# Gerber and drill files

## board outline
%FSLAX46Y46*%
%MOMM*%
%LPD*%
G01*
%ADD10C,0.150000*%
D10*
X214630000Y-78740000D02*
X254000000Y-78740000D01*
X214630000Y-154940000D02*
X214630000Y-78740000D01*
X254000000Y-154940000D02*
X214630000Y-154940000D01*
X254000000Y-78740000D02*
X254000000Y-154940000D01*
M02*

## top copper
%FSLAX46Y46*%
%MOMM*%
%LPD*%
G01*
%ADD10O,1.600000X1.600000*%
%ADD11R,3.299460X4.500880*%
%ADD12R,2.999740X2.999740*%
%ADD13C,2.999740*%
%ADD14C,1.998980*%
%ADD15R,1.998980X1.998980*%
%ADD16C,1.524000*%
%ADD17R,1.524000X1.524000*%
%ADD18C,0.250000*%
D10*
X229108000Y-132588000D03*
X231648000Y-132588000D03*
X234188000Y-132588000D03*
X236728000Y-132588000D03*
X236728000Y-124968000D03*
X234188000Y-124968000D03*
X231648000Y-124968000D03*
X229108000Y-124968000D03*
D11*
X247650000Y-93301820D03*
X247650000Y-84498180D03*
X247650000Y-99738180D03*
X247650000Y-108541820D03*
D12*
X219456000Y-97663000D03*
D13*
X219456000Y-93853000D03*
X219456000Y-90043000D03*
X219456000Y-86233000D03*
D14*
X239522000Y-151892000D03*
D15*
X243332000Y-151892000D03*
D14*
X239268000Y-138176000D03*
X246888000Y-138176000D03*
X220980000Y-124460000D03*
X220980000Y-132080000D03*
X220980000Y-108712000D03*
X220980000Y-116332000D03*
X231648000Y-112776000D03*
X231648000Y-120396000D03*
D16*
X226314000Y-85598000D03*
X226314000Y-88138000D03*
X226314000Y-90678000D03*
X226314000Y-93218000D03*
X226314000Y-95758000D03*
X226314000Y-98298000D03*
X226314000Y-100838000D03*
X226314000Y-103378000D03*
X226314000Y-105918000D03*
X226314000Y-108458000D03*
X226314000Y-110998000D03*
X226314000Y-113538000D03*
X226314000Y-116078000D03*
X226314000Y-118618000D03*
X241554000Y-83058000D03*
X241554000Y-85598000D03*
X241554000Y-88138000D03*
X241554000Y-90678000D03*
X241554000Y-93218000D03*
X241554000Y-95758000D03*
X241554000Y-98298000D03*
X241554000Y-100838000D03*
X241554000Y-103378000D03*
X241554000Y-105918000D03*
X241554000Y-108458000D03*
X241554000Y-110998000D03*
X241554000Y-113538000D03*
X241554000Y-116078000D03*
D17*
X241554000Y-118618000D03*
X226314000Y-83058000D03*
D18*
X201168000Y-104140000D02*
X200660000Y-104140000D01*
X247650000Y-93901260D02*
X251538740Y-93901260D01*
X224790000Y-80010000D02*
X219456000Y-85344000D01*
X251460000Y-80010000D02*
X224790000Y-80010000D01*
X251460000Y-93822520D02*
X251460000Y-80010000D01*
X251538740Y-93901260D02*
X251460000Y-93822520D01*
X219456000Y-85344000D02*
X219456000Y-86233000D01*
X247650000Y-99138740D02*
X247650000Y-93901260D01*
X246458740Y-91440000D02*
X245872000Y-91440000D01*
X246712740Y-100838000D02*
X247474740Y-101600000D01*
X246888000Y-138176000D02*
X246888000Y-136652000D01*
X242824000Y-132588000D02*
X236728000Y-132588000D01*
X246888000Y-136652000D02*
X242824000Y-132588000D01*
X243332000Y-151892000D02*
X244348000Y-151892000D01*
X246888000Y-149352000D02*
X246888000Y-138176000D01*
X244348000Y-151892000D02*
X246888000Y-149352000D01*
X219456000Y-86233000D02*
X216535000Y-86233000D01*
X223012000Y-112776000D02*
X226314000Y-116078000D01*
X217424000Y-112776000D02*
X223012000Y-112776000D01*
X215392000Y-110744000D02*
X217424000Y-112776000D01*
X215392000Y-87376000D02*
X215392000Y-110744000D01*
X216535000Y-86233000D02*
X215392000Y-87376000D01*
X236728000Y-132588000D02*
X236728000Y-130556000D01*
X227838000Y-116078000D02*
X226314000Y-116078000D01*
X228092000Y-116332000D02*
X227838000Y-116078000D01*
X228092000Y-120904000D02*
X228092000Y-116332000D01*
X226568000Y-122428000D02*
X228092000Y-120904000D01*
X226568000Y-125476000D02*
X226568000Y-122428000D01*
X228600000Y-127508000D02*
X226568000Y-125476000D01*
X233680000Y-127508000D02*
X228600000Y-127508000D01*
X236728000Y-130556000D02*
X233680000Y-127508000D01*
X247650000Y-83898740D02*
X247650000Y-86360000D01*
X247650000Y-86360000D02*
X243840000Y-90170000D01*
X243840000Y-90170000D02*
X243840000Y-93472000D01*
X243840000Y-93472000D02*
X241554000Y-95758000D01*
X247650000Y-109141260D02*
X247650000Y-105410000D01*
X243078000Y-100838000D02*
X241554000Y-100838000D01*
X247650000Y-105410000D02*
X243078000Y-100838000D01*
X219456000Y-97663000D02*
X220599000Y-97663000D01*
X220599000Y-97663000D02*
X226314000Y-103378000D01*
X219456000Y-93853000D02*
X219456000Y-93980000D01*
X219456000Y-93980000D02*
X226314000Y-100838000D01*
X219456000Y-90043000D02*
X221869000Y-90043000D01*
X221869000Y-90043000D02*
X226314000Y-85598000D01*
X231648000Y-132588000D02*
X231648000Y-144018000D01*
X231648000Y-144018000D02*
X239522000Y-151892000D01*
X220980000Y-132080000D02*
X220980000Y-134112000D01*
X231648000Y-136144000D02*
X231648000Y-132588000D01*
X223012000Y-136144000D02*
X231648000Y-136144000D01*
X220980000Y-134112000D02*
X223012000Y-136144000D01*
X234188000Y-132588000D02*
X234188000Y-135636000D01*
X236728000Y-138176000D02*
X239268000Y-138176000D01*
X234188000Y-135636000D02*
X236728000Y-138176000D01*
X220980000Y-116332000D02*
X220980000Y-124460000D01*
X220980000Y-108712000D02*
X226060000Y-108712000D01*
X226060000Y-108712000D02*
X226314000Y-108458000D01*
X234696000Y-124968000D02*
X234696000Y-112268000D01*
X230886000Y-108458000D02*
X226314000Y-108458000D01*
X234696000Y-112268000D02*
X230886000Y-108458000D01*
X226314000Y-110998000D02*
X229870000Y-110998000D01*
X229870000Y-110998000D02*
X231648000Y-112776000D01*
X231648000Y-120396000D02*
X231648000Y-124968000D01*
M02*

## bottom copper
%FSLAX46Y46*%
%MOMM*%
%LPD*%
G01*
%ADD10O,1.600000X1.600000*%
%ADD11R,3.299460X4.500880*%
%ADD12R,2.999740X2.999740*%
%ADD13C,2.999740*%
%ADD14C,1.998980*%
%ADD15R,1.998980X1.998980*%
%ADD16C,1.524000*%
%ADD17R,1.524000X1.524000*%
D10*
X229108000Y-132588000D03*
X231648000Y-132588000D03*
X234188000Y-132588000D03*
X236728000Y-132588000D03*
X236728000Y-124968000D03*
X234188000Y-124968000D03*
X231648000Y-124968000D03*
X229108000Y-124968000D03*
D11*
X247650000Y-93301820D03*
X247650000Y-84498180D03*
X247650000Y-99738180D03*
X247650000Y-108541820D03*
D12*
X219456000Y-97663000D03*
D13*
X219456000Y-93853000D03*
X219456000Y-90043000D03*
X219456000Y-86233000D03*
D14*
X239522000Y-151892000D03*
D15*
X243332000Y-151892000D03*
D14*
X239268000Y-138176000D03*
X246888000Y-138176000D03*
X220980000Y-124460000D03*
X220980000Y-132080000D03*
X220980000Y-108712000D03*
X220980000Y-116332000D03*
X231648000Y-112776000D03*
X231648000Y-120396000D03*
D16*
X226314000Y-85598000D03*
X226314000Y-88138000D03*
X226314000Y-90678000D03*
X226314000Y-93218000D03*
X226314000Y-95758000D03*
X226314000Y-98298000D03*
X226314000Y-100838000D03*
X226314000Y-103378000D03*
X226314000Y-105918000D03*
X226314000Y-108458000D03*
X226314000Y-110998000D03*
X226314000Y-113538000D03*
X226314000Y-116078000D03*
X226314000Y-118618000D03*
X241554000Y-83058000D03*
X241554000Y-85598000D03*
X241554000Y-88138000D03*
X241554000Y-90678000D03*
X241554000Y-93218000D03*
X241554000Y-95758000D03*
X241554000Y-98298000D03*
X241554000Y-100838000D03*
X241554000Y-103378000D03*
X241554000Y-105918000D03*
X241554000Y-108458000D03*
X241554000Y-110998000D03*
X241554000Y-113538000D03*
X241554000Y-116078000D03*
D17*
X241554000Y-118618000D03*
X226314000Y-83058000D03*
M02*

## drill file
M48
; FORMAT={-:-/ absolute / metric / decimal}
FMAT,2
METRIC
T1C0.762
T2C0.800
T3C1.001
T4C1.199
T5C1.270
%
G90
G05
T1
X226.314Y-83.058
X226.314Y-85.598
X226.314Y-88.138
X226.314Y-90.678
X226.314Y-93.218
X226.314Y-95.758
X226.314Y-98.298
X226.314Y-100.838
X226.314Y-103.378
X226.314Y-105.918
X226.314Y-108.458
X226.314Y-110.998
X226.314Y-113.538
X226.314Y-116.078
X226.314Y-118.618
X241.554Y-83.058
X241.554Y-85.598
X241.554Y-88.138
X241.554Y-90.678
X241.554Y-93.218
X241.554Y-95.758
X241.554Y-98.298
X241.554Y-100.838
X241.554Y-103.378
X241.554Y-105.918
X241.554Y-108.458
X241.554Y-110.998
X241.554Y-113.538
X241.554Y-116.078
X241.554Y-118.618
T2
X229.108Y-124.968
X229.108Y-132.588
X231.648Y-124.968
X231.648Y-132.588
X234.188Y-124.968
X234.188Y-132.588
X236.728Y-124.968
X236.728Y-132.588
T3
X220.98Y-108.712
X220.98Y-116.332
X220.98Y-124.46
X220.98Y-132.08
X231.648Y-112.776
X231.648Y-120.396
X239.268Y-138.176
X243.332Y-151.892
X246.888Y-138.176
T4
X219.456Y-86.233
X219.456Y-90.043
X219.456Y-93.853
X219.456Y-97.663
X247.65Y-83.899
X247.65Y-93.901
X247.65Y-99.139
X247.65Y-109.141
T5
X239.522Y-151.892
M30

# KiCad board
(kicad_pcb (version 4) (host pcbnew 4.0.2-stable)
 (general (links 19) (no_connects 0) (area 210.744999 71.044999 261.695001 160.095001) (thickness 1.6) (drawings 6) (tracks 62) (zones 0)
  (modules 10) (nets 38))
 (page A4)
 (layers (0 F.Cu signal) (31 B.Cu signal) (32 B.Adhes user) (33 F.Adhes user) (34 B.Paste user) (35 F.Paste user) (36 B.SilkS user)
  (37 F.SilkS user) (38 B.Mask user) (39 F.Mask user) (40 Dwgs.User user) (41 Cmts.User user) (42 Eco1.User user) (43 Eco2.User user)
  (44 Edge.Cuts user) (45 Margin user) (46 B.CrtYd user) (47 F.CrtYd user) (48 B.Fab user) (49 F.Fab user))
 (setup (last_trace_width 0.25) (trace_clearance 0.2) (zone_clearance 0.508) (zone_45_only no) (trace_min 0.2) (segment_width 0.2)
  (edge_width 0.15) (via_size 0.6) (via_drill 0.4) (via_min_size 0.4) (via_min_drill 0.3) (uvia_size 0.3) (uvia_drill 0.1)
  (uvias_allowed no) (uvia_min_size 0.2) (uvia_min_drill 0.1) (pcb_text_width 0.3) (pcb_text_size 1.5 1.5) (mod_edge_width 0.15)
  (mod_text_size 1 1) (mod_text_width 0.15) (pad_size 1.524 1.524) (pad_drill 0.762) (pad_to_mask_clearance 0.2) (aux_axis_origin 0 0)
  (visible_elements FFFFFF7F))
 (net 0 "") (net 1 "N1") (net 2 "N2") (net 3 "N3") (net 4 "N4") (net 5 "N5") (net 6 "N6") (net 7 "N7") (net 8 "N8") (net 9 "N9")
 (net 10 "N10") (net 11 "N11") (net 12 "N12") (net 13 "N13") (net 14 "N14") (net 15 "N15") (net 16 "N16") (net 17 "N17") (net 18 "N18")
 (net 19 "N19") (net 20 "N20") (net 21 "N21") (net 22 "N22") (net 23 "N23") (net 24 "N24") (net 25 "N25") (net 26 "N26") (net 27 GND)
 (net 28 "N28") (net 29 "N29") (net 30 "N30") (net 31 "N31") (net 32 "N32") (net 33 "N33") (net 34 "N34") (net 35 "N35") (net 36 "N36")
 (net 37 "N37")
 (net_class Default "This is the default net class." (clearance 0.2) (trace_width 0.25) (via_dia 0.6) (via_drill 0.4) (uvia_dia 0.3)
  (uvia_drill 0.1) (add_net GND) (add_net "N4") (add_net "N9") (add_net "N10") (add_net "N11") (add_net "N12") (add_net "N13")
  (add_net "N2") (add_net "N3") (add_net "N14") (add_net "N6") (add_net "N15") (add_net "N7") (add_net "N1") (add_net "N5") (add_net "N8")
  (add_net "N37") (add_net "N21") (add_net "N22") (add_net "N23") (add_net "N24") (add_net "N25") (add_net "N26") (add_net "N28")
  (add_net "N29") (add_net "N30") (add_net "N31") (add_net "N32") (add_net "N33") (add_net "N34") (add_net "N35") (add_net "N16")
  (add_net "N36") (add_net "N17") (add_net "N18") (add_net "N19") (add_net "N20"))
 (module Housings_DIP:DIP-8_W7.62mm (layer F.Cu) (at 229.108 132.588 90)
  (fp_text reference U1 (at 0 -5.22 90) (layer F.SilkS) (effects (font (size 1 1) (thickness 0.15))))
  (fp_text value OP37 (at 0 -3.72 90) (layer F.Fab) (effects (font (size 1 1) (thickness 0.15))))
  (pad 1 thru_hole oval (at 0 0 90) (size 1.6 1.6) (drill 0.8) (layers *.Cu *.Mask F.SilkS) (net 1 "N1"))
  (pad 2 thru_hole oval (at 0 2.54 90) (size 1.6 1.6) (drill 0.8) (layers *.Cu *.Mask F.SilkS) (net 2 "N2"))
  (pad 3 thru_hole oval (at 0 5.08 90) (size 1.6 1.6) (drill 0.8) (layers *.Cu *.Mask F.SilkS) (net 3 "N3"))
  (pad 4 thru_hole oval (at 0 7.62 90) (size 1.6 1.6) (drill 0.8) (layers *.Cu *.Mask F.SilkS) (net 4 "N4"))
  (pad 5 thru_hole oval (at 7.62 7.62 90) (size 1.6 1.6) (drill 0.8) (layers *.Cu *.Mask F.SilkS) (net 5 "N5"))
  (pad 6 thru_hole oval (at 7.62 5.08 90) (size 1.6 1.6) (drill 0.8) (layers *.Cu *.Mask F.SilkS) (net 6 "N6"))
  (pad 7 thru_hole oval (at 7.62 2.54 90) (size 1.6 1.6) (drill 0.8) (layers *.Cu *.Mask F.SilkS) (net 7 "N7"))
  (pad 8 thru_hole oval (at 7.62 0 90) (size 1.6 1.6) (drill 0.8) (layers *.Cu *.Mask F.SilkS) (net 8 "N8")))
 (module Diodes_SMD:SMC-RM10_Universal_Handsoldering (layer F.Cu) (at 247.65 88.9 90)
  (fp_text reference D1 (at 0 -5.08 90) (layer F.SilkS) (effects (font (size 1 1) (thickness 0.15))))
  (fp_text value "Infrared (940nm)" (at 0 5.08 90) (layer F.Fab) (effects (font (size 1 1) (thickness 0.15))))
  (pad 1 thru_hole rect (at -5.00126 0 90) (size 4.50088 3.29946) (drill 1.19888 (offset 0.59944 0)) (layers *.Cu *.Mask F.SilkS)
   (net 4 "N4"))
  (pad 2 thru_hole rect (at 5.00126 0 270) (size 4.50088 3.29946) (drill 1.19888 (offset 0.59944 0)) (layers *.Cu *.Mask F.SilkS)
   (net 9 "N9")))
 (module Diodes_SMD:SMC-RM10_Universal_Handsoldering (layer F.Cu) (at 247.65 104.14 270)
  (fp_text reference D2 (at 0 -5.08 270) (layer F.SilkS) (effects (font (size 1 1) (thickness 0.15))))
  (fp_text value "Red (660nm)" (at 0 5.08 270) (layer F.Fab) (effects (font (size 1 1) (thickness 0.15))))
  (pad 1 thru_hole rect (at -5.00126 0 270) (size 4.50088 3.29946) (drill 1.19888 (offset 0.59944 0)) (layers *.Cu *.Mask F.SilkS)
   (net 4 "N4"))
  (pad 2 thru_hole rect (at 5.00126 0 90) (size 4.50088 3.29946) (drill 1.19888 (offset 0.59944 0)) (layers *.Cu *.Mask F.SilkS)
   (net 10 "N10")))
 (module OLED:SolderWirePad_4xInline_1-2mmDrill (layer F.Cu) (at 219.456 91.948 90)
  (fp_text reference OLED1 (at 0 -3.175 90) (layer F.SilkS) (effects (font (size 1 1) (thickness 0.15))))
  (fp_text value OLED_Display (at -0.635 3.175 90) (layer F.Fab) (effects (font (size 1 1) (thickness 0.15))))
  (pad 1 thru_hole rect (at -5.715 0 90) (size 2.99974 2.99974) (drill 1.19888) (layers *.Cu *.Mask F.SilkS) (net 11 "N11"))
  (pad 2 thru_hole circle (at -1.905 0 90) (size 2.99974 2.99974) (drill 1.19888) (layers *.Cu *.Mask F.SilkS) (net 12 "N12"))
  (pad 3 thru_hole circle (at 1.905 0 90) (size 2.99974 2.99974) (drill 1.19888) (layers *.Cu *.Mask F.SilkS) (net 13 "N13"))
  (pad 4 thru_hole circle (at 5.715 0 90) (size 2.99974 2.99974) (drill 1.19888) (layers *.Cu *.Mask F.SilkS) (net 4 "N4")))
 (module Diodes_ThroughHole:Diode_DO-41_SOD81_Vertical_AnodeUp (layer F.Cu) (at 243.332 151.892 180)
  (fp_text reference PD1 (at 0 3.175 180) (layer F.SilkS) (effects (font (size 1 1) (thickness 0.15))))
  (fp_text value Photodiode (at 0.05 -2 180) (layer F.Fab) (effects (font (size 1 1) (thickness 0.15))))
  (pad 2 thru_hole circle (at 3.81 0 180) (size 1.99898 1.99898) (drill 1.27) (layers *.Cu *.Mask F.SilkS) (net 2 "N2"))
  (pad 1 thru_hole rect (at 0 0 180) (size 1.99898 1.99898) (drill 1.00076) (layers *.Cu *.Mask F.SilkS) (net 4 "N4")))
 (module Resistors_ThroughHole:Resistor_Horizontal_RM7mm (layer F.Cu) (at 239.268 138.176)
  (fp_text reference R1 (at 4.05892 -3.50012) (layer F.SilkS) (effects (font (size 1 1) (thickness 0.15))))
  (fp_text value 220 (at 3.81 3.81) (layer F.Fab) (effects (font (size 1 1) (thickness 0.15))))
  (pad 1 thru_hole circle (at 0 0) (size 1.99898 1.99898) (drill 1.00076) (layers *.Cu *.SilkS *.Mask) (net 3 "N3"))
  (pad 2 thru_hole circle (at 7.62 0) (size 1.99898 1.99898) (drill 1.00076) (layers *.Cu *.SilkS *.Mask) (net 4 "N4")))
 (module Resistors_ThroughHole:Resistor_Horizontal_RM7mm (layer F.Cu) (at 220.98 124.46 270)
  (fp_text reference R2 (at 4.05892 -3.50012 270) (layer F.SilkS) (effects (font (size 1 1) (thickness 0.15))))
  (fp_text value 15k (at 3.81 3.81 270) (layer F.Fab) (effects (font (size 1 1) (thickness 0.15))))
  (pad 1 thru_hole circle (at 0 0 270) (size 1.99898 1.99898) (drill 1.00076) (layers *.Cu *.SilkS *.Mask) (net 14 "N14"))
  (pad 2 thru_hole circle (at 7.62 0 270) (size 1.99898 1.99898) (drill 1.00076) (layers *.Cu *.SilkS *.Mask) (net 2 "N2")))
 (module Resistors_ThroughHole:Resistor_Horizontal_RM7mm (layer F.Cu) (at 220.98 108.712 270)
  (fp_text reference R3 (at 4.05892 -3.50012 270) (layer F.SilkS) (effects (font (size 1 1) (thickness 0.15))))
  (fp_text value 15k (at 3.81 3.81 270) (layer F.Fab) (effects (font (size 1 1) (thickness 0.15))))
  (pad 1 thru_hole circle (at 0 0 270) (size 1.99898 1.99898) (drill 1.00076) (layers *.Cu *.SilkS *.Mask) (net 6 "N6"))
  (pad 2 thru_hole circle (at 7.62 0 270) (size 1.99898 1.99898) (drill 1.00076) (layers *.Cu *.SilkS *.Mask) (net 14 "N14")))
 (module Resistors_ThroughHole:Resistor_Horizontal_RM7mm (layer F.Cu) (at 231.648 112.776 270)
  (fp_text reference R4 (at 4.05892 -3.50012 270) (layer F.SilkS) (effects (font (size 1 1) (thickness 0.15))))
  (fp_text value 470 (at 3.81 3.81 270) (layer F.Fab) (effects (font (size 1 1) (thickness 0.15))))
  (pad 1 thru_hole circle (at 0 0 270) (size 1.99898 1.99898) (drill 1.00076) (layers *.Cu *.SilkS *.Mask) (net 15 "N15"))
  (pad 2 thru_hole circle (at 7.62 0 270) (size 1.99898 1.99898) (drill 1.00076) (layers *.Cu *.SilkS *.Mask) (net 7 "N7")))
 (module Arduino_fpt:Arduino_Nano (layer F.Cu) (at 243.332 79.248 270)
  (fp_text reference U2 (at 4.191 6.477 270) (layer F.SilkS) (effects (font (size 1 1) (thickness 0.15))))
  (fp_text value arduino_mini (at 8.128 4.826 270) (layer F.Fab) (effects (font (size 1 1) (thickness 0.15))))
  (pad 2 thru_hole circle (at 6.35 17.018 270) (size 1.524 1.524) (drill 0.762) (layers *.Cu *.Mask F.SilkS) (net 13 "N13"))
  (pad 3 thru_hole circle (at 8.89 17.018 270) (size 1.524 1.524) (drill 0.762) (layers *.Cu *.Mask F.SilkS) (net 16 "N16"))
  (pad 4 thru_hole circle (at 11.43 17.018 270) (size 1.524 1.524) (drill 0.762) (layers *.Cu *.Mask F.SilkS) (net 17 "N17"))
  (pad 5 thru_hole circle (at 13.97 17.018 270) (size 1.524 1.524) (drill 0.762) (layers *.Cu *.Mask F.SilkS) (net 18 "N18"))
  (pad 6 thru_hole circle (at 16.51 17.018 270) (size 1.524 1.524) (drill 0.762) (layers *.Cu *.Mask F.SilkS) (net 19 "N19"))
  (pad 7 thru_hole circle (at 19.05 17.018 270) (size 1.524 1.524) (drill 0.762) (layers *.Cu *.Mask F.SilkS) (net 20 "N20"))
  (pad 8 thru_hole circle (at 21.59 17.018 270) (size 1.524 1.524) (drill 0.762) (layers *.Cu *.Mask F.SilkS) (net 12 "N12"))
  (pad 9 thru_hole circle (at 24.13 17.018 270) (size 1.524 1.524) (drill 0.762) (layers *.Cu *.Mask F.SilkS) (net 11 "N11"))
  (pad 10 thru_hole circle (at 26.67 17.018 270) (size 1.524 1.524) (drill 0.762) (layers *.Cu *.Mask F.SilkS) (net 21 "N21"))
  (pad 11 thru_hole circle (at 29.21 17.018 270) (size 1.524 1.524) (drill 0.762) (layers *.Cu *.Mask F.SilkS) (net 6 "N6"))
  (pad 12 thru_hole circle (at 31.75 17.018 270) (size 1.524 1.524) (drill 0.762) (layers *.Cu *.Mask F.SilkS) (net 15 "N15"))
  (pad 13 thru_hole circle (at 34.29 17.018 270) (size 1.524 1.524) (drill 0.762) (layers *.Cu *.Mask F.SilkS) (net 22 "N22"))
  (pad 14 thru_hole circle (at 36.83 17.018 270) (size 1.524 1.524) (drill 0.762) (layers *.Cu *.Mask F.SilkS) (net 4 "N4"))
  (pad 15 thru_hole circle (at 39.37 17.018 270) (size 1.524 1.524) (drill 0.762) (layers *.Cu *.Mask F.SilkS) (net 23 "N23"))
  (pad 16 thru_hole circle (at 3.81 1.778 270) (size 1.524 1.524) (drill 0.762) (layers *.Cu *.Mask F.SilkS) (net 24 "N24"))
  (pad 17 thru_hole circle (at 6.35 1.778 270) (size 1.524 1.524) (drill 0.762) (layers *.Cu *.Mask F.SilkS) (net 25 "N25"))
  (pad 18 thru_hole circle (at 8.89 1.778 270) (size 1.524 1.524) (drill 0.762) (layers *.Cu *.Mask F.SilkS) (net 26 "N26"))
  (pad 19 thru_hole circle (at 11.43 1.778 270) (size 1.524 1.524) (drill 0.762) (layers *.Cu *.Mask F.SilkS) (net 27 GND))
  (pad 20 thru_hole circle (at 13.97 1.778 270) (size 1.524 1.524) (drill 0.762) (layers *.Cu *.Mask F.SilkS) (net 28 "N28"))
  (pad 21 thru_hole circle (at 16.51 1.778 270) (size 1.524 1.524) (drill 0.762) (layers *.Cu *.Mask F.SilkS) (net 9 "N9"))
  (pad 22 thru_hole circle (at 19.05 1.778 270) (size 1.524 1.524) (drill 0.762) (layers *.Cu *.Mask F.SilkS) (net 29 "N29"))
  (pad 23 thru_hole circle (at 21.59 1.778 270) (size 1.524 1.524) (drill 0.762) (layers *.Cu *.Mask F.SilkS) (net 10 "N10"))
  (pad 24 thru_hole circle (at 24.13 1.778 270) (size 1.524 1.524) (drill 0.762) (layers *.Cu *.Mask F.SilkS) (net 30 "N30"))
  (pad 25 thru_hole circle (at 26.67 1.778 270) (size 1.524 1.524) (drill 0.762) (layers *.Cu *.Mask F.SilkS) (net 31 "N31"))
  (pad 26 thru_hole circle (at 29.21 1.778 270) (size 1.524 1.524) (drill 0.762) (layers *.Cu *.Mask F.SilkS) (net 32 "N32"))
  (pad 27 thru_hole circle (at 31.75 1.778 270) (size 1.524 1.524) (drill 0.762) (layers *.Cu *.Mask F.SilkS) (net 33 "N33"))
  (pad 28 thru_hole circle (at 34.29 1.778 270) (size 1.524 1.524) (drill 0.762) (layers *.Cu *.Mask F.SilkS) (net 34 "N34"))
  (pad 29 thru_hole circle (at 36.83 1.778 270) (size 1.524 1.524) (drill 0.762) (layers *.Cu *.Mask F.SilkS) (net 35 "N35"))
  (pad 30 thru_hole rect (at 39.37 1.778 270) (size 1.524 1.524) (drill 0.762) (layers *.Cu *.Mask F.SilkS) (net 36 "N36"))
  (pad 1 thru_hole rect (at 3.81 17.018 270) (size 1.524 1.524) (drill 0.762) (layers *.Cu *.Mask F.SilkS) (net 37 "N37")))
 (gr_line (start 214.63 78.74) (end 254 78.74) (angle 90) (layer Edge.Cuts) (width 0.15))
 (gr_line (start 214.63 154.94) (end 214.63 78.74) (angle 90) (layer Edge.Cuts) (width 0.15))
 (gr_line (start 254 154.94) (end 214.63 154.94) (angle 90) (layer Edge.Cuts) (width 0.15))
 (gr_line (start 254 78.74) (end 254 154.94) (angle 90) (layer Edge.Cuts) (width 0.15))
 (segment (start 201.168 104.14) (end 200.66 104.14) (width 0.25) (layer F.Cu) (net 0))
 (segment (start 247.65 93.90126) (end 251.53874 93.90126) (width 0.25) (layer F.Cu) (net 4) (status 400000))
 (segment (start 224.79 80.01) (end 219.456 85.344) (width 0.25) (layer F.Cu) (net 4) (status 800000))
 (segment (start 251.46 80.01) (end 224.79 80.01) (width 0.25) (layer F.Cu) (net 4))
 (segment (start 251.46 93.82252) (end 251.46 80.01) (width 0.25) (layer F.Cu) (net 4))
 (segment (start 251.53874 93.90126) (end 251.46 93.82252) (width 0.25) (layer F.Cu) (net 4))
 (segment (start 219.456 85.344) (end 219.456 86.233) (width 0.25) (layer F.Cu) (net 4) (status C00000))
 (segment (start 247.65 99.13874) (end 247.65 93.90126) (width 0.25) (layer F.Cu) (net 4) (status C00000))
 (segment (start 246.45874 91.44) (end 245.872 91.44) (width 0.25) (layer F.Cu) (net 4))
 (segment (start 246.71274 100.838) (end 247.47474 101.6) (width 0.25) (layer F.Cu) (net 4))
 (segment (start 246.888 138.176) (end 246.888 136.652) (width 0.25) (layer F.Cu) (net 4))
 (segment (start 242.824 132.588) (end 236.728 132.588) (width 0.25) (layer F.Cu) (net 4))
 (segment (start 246.888 136.652) (end 242.824 132.588) (width 0.25) (layer F.Cu) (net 4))
 (segment (start 243.332 151.892) (end 244.348 151.892) (width 0.25) (layer F.Cu) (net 4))
 (segment (start 246.888 149.352) (end 246.888 138.176) (width 0.25) (layer F.Cu) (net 4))
 (segment (start 244.348 151.892) (end 246.888 149.352) (width 0.25) (layer F.Cu) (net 4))
 (segment (start 219.456 86.233) (end 216.535 86.233) (width 0.25) (layer F.Cu) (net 4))
 (segment (start 223.012 112.776) (end 226.314 116.078) (width 0.25) (layer F.Cu) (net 4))
 (segment (start 217.424 112.776) (end 223.012 112.776) (width 0.25) (layer F.Cu) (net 4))
 (segment (start 215.392 110.744) (end 217.424 112.776) (width 0.25) (layer F.Cu) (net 4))
 (segment (start 215.392 87.376) (end 215.392 110.744) (width 0.25) (layer F.Cu) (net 4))
 (segment (start 216.535 86.233) (end 215.392 87.376) (width 0.25) (layer F.Cu) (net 4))
 (segment (start 236.728 132.588) (end 236.728 130.556) (width 0.25) (layer F.Cu) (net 4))
 (segment (start 227.838 116.078) (end 226.314 116.078) (width 0.25) (layer F.Cu) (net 4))
 (segment (start 228.092 116.332) (end 227.838 116.078) (width 0.25) (layer F.Cu) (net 4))
 (segment (start 228.092 120.904) (end 228.092 116.332) (width 0.25) (layer F.Cu) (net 4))
 (segment (start 226.568 122.428) (end 228.092 120.904) (width 0.25) (layer F.Cu) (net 4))
 (segment (start 226.568 125.476) (end 226.568 122.428) (width 0.25) (layer F.Cu) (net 4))
 (segment (start 228.6 127.508) (end 226.568 125.476) (width 0.25) (layer F.Cu) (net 4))
 (segment (start 233.68 127.508) (end 228.6 127.508) (width 0.25) (layer F.Cu) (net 4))
 (segment (start 236.728 130.556) (end 233.68 127.508) (width 0.25) (layer F.Cu) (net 4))
 (segment (start 247.65 83.89874) (end 247.65 86.36) (width 0.25) (layer F.Cu) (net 9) (status C00000))
 (segment (start 247.65 86.36) (end 243.84 90.17) (width 0.25) (layer F.Cu) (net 9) (status 400000))
 (segment (start 243.84 90.17) (end 243.84 93.472) (width 0.25) (layer F.Cu) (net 9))
 (segment (start 243.84 93.472) (end 241.554 95.758) (width 0.25) (layer F.Cu) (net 9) (status 800000))
 (segment (start 247.65 109.14126) (end 247.65 105.41) (width 0.25) (layer F.Cu) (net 10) (status 400000))
 (segment (start 243.078 100.838) (end 241.554 100.838) (width 0.25) (layer F.Cu) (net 10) (status 800000))
 (segment (start 247.65 105.41) (end 243.078 100.838) (width 0.25) (layer F.Cu) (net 10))
 (segment (start 219.456 97.663) (end 220.599 97.663) (width 0.25) (layer F.Cu) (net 11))
 (segment (start 220.599 97.663) (end 226.314 103.378) (width 0.25) (layer F.Cu) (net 11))
 (segment (start 219.456 93.853) (end 219.456 93.98) (width 0.25) (layer F.Cu) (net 12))
 (segment (start 219.456 93.98) (end 226.314 100.838) (width 0.25) (layer F.Cu) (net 12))
 (segment (start 219.456 90.043) (end 221.869 90.043) (width 0.25) (layer F.Cu) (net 13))
 (segment (start 221.869 90.043) (end 226.314 85.598) (width 0.25) (layer F.Cu) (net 13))
 (segment (start 231.648 132.588) (end 231.648 144.018) (width 0.25) (layer F.Cu) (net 2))
 (segment (start 231.648 144.018) (end 239.522 151.892) (width 0.25) (layer F.Cu) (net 2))
 (segment (start 220.98 132.08) (end 220.98 134.112) (width 0.25) (layer F.Cu) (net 2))
 (segment (start 231.648 136.144) (end 231.648 132.588) (width 0.25) (layer F.Cu) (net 2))
 (segment (start 223.012 136.144) (end 231.648 136.144) (width 0.25) (layer F.Cu) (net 2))
 (segment (start 220.98 134.112) (end 223.012 136.144) (width 0.25) (layer F.Cu) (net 2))
 (segment (start 234.188 132.588) (end 234.188 135.636) (width 0.25) (layer F.Cu) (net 3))
 (segment (start 236.728 138.176) (end 239.268 138.176) (width 0.25) (layer F.Cu) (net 3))
 (segment (start 234.188 135.636) (end 236.728 138.176) (width 0.25) (layer F.Cu) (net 3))
 (segment (start 220.98 116.332) (end 220.98 124.46) (width 0.25) (layer F.Cu) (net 14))
 (segment (start 220.98 108.712) (end 226.06 108.712) (width 0.25) (layer F.Cu) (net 6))
 (segment (start 226.06 108.712) (end 226.314 108.458) (width 0.25) (layer F.Cu) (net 6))
 (segment (start 234.696 124.968) (end 234.696 112.268) (width 0.25) (layer F.Cu) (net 6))
 (segment (start 230.886 108.458) (end 226.314 108.458) (width 0.25) (layer F.Cu) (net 6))
 (segment (start 234.696 112.268) (end 230.886 108.458) (width 0.25) (layer F.Cu) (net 6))
 (segment (start 226.314 110.998) (end 229.87 110.998) (width 0.25) (layer F.Cu) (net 15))
 (segment (start 229.87 110.998) (end 231.648 112.776) (width 0.25) (layer F.Cu) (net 15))
 (segment (start 231.648 120.396) (end 231.648 124.968) (width 0.25) (layer F.Cu) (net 7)))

